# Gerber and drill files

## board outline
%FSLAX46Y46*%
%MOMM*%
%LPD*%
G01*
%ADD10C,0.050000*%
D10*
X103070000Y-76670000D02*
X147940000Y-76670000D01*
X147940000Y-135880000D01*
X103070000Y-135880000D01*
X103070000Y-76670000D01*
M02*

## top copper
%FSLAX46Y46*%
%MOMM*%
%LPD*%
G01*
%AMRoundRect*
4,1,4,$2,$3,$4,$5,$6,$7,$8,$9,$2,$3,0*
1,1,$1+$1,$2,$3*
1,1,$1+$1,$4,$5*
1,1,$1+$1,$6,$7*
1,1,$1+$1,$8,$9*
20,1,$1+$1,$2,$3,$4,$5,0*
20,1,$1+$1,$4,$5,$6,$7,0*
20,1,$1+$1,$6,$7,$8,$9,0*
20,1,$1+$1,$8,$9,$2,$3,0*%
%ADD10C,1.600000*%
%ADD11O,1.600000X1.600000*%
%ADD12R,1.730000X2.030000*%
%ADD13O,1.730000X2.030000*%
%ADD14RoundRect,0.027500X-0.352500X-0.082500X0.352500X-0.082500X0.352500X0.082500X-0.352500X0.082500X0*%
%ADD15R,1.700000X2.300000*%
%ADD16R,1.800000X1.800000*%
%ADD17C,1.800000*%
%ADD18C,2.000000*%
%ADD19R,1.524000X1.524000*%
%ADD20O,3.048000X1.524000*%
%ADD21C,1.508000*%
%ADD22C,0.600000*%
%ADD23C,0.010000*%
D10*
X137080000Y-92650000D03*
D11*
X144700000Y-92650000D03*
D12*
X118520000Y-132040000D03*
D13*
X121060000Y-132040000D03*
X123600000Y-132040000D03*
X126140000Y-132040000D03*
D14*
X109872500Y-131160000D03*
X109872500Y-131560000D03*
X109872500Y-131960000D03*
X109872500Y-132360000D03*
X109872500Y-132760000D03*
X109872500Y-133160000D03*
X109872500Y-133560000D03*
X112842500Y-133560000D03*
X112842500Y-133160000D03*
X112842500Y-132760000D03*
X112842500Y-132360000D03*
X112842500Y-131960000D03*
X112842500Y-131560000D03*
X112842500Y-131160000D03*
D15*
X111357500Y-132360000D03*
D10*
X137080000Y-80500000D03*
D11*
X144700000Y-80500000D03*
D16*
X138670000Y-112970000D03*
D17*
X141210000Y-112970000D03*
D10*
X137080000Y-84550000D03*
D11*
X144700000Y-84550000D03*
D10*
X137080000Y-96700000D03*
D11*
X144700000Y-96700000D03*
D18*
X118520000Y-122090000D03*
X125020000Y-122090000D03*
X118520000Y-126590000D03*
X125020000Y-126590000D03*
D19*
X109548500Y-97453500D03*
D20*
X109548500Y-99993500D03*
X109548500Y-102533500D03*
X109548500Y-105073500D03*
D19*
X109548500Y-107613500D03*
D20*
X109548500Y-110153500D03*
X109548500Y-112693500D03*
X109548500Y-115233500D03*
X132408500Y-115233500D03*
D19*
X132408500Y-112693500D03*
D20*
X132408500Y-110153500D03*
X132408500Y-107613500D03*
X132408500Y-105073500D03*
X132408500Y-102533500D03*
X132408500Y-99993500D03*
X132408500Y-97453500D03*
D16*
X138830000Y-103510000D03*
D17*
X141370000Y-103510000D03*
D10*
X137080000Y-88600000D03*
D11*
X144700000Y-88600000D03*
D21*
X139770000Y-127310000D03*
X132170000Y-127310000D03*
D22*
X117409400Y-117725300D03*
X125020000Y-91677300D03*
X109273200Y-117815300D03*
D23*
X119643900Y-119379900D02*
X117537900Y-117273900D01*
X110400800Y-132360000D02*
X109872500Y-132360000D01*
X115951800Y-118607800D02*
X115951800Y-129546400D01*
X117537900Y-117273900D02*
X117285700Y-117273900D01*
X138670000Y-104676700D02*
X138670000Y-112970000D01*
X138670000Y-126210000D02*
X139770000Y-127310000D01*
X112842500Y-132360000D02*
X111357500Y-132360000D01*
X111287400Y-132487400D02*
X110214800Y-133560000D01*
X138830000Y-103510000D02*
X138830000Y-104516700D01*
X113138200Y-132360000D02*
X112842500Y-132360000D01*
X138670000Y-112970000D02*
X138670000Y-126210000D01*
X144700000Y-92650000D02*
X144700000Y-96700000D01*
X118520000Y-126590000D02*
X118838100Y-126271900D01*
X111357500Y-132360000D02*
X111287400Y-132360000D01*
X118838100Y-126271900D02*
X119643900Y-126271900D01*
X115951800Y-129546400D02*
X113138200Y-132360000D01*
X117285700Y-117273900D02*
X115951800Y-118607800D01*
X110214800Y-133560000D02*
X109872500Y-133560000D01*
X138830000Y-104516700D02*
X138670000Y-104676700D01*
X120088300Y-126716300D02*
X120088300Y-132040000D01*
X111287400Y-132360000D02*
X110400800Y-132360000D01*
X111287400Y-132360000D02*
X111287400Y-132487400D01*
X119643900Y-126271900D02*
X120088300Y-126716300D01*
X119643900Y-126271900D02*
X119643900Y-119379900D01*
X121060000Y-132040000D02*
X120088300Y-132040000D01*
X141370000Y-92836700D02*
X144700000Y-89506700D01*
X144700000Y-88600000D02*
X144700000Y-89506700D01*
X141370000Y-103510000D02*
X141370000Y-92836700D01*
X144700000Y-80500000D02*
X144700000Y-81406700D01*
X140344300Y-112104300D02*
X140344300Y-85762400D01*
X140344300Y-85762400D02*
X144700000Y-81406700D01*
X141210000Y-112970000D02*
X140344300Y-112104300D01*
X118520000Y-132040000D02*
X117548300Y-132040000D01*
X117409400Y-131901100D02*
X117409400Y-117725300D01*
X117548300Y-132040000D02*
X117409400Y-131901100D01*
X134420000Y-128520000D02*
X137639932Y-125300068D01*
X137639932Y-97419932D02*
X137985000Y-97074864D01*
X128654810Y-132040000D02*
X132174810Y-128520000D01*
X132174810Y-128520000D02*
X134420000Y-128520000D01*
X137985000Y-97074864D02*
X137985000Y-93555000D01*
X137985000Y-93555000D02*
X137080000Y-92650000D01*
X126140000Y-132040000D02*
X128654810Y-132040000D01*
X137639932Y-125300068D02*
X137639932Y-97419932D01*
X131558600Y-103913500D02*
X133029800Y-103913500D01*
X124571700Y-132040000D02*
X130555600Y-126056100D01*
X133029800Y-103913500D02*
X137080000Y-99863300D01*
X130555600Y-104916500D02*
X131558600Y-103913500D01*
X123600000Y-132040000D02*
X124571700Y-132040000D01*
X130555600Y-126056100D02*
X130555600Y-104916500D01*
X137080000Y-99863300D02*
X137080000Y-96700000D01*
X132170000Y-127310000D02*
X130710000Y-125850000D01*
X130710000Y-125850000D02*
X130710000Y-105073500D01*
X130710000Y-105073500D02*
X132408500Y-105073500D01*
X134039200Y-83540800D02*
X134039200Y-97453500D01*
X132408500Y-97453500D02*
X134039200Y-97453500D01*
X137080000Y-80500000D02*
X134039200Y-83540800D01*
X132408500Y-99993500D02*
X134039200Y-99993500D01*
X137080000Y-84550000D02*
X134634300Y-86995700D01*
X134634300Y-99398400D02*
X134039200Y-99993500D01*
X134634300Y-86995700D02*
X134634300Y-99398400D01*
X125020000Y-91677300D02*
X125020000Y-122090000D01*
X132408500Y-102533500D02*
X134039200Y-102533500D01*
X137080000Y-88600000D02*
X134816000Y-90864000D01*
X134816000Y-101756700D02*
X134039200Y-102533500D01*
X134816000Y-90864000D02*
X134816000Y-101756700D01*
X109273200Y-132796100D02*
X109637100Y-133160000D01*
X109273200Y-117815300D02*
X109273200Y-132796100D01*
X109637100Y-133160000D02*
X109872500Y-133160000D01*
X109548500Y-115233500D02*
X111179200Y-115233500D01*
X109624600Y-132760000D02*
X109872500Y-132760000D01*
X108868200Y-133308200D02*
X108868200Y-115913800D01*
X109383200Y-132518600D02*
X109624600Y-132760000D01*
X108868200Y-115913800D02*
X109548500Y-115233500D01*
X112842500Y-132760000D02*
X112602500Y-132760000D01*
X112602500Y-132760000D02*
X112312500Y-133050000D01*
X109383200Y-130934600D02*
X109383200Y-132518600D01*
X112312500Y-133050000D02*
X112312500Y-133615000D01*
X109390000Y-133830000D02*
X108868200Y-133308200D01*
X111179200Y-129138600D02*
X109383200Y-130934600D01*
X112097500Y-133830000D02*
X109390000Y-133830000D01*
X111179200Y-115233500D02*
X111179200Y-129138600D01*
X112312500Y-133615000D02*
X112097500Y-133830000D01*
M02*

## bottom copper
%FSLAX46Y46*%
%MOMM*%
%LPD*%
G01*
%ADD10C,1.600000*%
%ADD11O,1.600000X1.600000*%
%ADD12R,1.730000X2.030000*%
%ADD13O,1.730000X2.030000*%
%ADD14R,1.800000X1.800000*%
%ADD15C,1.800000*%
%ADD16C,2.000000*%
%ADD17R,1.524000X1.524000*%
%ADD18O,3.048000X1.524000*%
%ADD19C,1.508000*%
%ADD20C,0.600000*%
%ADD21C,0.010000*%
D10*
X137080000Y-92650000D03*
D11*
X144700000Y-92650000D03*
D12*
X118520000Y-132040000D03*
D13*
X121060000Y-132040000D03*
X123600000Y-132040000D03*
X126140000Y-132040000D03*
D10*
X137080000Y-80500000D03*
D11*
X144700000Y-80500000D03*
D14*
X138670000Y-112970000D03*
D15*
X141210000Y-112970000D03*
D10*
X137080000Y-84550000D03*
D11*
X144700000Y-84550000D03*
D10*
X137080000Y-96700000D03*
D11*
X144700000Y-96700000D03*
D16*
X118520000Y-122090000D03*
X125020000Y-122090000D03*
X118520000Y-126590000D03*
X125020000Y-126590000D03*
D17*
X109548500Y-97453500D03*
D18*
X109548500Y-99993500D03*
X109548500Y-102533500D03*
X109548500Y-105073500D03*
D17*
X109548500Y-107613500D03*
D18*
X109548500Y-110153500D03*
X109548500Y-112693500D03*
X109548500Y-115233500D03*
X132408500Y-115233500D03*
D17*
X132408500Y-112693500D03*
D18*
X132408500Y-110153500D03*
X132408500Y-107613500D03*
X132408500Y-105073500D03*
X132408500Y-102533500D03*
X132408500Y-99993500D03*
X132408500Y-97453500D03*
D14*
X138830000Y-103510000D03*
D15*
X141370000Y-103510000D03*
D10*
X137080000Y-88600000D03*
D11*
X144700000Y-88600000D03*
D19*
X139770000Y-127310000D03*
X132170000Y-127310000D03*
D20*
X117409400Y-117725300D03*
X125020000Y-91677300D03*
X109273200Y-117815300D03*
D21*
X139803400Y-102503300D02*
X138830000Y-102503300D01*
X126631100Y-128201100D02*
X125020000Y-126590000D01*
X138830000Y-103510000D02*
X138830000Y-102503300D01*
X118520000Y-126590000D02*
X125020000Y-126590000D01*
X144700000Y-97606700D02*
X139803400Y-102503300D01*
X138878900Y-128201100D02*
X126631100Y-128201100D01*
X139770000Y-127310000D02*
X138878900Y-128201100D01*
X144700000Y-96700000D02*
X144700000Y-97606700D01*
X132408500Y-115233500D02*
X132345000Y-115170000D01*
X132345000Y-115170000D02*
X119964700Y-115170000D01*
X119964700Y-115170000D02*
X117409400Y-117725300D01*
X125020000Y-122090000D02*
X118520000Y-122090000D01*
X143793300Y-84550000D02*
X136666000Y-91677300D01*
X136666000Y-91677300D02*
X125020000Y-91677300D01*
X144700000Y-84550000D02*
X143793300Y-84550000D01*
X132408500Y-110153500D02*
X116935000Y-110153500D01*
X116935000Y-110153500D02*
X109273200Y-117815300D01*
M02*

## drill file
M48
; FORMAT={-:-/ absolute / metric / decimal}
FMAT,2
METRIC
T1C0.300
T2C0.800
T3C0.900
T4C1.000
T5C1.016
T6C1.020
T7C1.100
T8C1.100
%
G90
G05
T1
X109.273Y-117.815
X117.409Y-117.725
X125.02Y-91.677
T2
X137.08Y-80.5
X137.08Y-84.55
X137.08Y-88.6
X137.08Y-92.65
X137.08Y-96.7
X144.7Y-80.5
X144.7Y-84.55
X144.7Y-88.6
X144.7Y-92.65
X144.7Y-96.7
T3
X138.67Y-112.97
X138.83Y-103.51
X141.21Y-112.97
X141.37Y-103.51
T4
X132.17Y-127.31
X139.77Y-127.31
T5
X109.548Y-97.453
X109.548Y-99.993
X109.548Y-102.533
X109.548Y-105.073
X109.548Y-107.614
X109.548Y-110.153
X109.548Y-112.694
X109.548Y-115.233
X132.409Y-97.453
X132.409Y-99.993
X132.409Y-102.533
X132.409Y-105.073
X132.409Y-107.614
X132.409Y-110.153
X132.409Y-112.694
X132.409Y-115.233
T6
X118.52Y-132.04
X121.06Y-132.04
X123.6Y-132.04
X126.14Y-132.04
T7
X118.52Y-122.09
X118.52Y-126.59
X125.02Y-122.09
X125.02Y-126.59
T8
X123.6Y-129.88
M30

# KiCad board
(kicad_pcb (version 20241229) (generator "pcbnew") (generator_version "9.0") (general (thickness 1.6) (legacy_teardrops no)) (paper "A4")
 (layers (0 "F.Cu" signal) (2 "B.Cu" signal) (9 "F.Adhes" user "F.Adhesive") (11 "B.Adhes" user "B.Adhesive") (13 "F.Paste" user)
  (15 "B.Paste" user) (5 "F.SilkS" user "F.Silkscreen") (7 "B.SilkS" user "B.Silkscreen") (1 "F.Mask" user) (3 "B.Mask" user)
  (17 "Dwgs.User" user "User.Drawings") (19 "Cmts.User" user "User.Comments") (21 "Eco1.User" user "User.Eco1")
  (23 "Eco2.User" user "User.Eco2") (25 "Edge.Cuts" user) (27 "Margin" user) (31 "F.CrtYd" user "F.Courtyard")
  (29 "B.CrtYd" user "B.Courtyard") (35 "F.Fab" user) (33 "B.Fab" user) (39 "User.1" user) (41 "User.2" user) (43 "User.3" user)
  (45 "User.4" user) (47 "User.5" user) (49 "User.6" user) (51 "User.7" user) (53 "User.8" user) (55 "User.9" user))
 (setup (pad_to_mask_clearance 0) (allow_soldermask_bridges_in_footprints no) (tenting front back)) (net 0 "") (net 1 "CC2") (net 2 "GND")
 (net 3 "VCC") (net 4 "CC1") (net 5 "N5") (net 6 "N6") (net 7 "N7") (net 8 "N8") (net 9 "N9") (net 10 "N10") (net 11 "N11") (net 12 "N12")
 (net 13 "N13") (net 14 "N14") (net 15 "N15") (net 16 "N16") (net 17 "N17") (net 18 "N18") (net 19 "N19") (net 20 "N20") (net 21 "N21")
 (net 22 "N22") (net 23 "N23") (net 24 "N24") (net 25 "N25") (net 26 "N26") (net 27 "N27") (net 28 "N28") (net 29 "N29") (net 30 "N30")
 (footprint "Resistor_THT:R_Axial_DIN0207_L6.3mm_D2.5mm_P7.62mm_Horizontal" (layer "F.Cu") (at 137.08 92.65)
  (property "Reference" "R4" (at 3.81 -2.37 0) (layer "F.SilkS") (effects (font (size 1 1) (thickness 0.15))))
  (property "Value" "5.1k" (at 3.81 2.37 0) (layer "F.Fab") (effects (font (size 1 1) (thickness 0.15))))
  (pad "1" thru_hole circle (at 0 0) (size 1.6 1.6) (drill 0.8) (layers "*.Cu" "*.Mask") (remove_unused_layers no) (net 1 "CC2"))
  (pad "2" thru_hole oval (at 7.62 0) (size 1.6 1.6) (drill 0.8) (layers "*.Cu" "*.Mask") (remove_unused_layers no) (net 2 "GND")))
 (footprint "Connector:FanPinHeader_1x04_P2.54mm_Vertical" (layer "F.Cu") (at 118.52 132.04)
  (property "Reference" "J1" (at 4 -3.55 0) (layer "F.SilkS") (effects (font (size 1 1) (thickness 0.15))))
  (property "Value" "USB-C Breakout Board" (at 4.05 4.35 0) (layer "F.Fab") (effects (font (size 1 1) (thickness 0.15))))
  (pad "" np_thru_hole circle (at 5.08 -2.16 90) (size 1.1 1.1) (drill 1.1) (layers "*.Cu" "*.Mask"))
  (pad "1" thru_hole rect (at 0 0 90) (size 2.03 1.73) (drill 1.02) (layers "*.Cu" "*.Mask") (remove_unused_layers no) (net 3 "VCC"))
  (pad "2" thru_hole oval (at 2.54 0 90) (size 2.03 1.73) (drill 1.02) (layers "*.Cu" "*.Mask") (remove_unused_layers no) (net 2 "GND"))
  (pad "3" thru_hole oval (at 5.08 0 90) (size 2.03 1.73) (drill 1.02) (layers "*.Cu" "*.Mask") (remove_unused_layers no) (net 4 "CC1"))
  (pad "4" thru_hole oval (at 7.62 0 90) (size 2.03 1.73) (drill 1.02) (layers "*.Cu" "*.Mask") (remove_unused_layers no) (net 1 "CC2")))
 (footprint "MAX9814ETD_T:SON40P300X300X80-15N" (layer "F.Cu") (at 111.3575 132.36)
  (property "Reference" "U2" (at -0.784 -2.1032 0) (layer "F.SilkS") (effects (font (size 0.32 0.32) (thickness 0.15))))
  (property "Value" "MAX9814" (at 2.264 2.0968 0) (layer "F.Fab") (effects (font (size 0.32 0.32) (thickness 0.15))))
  (pad "1" smd roundrect (at -1.485 -1.2) (size 0.76 0.22) (layers "F.Cu" "F.Mask" "F.Paste") (roundrect_rratio 0.125) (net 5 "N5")
   (solder_mask_margin 0.102))
  (pad "2" smd roundrect (at -1.485 -0.8) (size 0.76 0.22) (layers "F.Cu" "F.Mask" "F.Paste") (roundrect_rratio 0.125) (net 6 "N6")
   (solder_mask_margin 0.102))
  (pad "3" smd roundrect (at -1.485 -0.4) (size 0.76 0.22) (layers "F.Cu" "F.Mask" "F.Paste") (roundrect_rratio 0.125) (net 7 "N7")
   (solder_mask_margin 0.102))
  (pad "4" smd roundrect (at -1.485 0) (size 0.76 0.22) (layers "F.Cu" "F.Mask" "F.Paste") (roundrect_rratio 0.125) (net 2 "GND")
   (solder_mask_margin 0.102))
  (pad "5" smd roundrect (at -1.485 0.4) (size 0.76 0.22) (layers "F.Cu" "F.Mask" "F.Paste") (roundrect_rratio 0.125) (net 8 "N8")
   (solder_mask_margin 0.102))
  (pad "6" smd roundrect (at -1.485 0.8) (size 0.76 0.22) (layers "F.Cu" "F.Mask" "F.Paste") (roundrect_rratio 0.125) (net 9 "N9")
   (solder_mask_margin 0.102))
  (pad "7" smd roundrect (at -1.485 1.2) (size 0.76 0.22) (layers "F.Cu" "F.Mask" "F.Paste") (roundrect_rratio 0.125) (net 2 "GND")
   (solder_mask_margin 0.102))
  (pad "8" smd roundrect (at 1.485 1.2) (size 0.76 0.22) (layers "F.Cu" "F.Mask" "F.Paste") (roundrect_rratio 0.125) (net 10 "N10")
   (solder_mask_margin 0.102))
  (pad "9" smd roundrect (at 1.485 0.8) (size 0.76 0.22) (layers "F.Cu" "F.Mask" "F.Paste") (roundrect_rratio 0.125) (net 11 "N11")
   (solder_mask_margin 0.102))
  (pad "10" smd roundrect (at 1.485 0.4) (size 0.76 0.22) (layers "F.Cu" "F.Mask" "F.Paste") (roundrect_rratio 0.125) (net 8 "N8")
   (solder_mask_margin 0.102))
  (pad "11" smd roundrect (at 1.485 0) (size 0.76 0.22) (layers "F.Cu" "F.Mask" "F.Paste") (roundrect_rratio 0.125) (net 2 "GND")
   (solder_mask_margin 0.102))
  (pad "12" smd roundrect (at 1.485 -0.4) (size 0.76 0.22) (layers "F.Cu" "F.Mask" "F.Paste") (roundrect_rratio 0.125) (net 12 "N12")
   (solder_mask_margin 0.102))
  (pad "13" smd roundrect (at 1.485 -0.8) (size 0.76 0.22) (layers "F.Cu" "F.Mask" "F.Paste") (roundrect_rratio 0.125) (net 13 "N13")
   (solder_mask_margin 0.102))
  (pad "14" smd roundrect (at 1.485 -1.2) (size 0.76 0.22) (layers "F.Cu" "F.Mask" "F.Paste") (roundrect_rratio 0.125) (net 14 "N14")
   (solder_mask_margin 0.102))
  (pad "15" smd rect (at 0 0) (size 1.7 2.3) (layers "F.Cu" "F.Mask") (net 2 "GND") (solder_mask_margin 0.102)))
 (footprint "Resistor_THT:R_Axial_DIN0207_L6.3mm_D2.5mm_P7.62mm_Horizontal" (layer "F.Cu") (at 137.08 80.5)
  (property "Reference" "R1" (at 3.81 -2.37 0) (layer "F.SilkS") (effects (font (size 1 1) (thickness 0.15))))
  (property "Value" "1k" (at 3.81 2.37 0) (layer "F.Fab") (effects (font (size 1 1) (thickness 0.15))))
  (pad "1" thru_hole circle (at 0 0) (size 1.6 1.6) (drill 0.8) (layers "*.Cu" "*.Mask") (remove_unused_layers no) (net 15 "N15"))
  (pad "2" thru_hole oval (at 7.62 0) (size 1.6 1.6) (drill 0.8) (layers "*.Cu" "*.Mask") (remove_unused_layers no) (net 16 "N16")))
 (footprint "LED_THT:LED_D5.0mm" (layer "F.Cu") (at 138.67 112.97)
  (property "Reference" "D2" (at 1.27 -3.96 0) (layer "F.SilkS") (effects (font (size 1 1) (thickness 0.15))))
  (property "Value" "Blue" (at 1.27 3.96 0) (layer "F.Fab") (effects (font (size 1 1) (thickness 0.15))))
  (pad "1" thru_hole rect (at 0 0) (size 1.8 1.8) (drill 0.9) (layers "*.Cu" "*.Mask") (remove_unused_layers no) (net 2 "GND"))
  (pad "2" thru_hole circle (at 2.54 0) (size 1.8 1.8) (drill 0.9) (layers "*.Cu" "*.Mask") (remove_unused_layers no) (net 16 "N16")))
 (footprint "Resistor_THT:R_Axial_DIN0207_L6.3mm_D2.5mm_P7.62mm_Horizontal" (layer "F.Cu") (at 137.08 84.55)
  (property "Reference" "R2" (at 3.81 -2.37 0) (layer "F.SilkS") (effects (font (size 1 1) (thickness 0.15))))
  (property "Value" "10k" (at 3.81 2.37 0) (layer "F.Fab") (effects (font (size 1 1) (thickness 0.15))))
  (pad "1" thru_hole circle (at 0 0) (size 1.6 1.6) (drill 0.8) (layers "*.Cu" "*.Mask") (remove_unused_layers no) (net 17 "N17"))
  (pad "2" thru_hole oval (at 7.62 0) (size 1.6 1.6) (drill 0.8) (layers "*.Cu" "*.Mask") (remove_unused_layers no) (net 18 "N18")))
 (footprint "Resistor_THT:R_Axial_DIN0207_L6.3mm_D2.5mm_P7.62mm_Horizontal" (layer "F.Cu") (at 137.08 96.7)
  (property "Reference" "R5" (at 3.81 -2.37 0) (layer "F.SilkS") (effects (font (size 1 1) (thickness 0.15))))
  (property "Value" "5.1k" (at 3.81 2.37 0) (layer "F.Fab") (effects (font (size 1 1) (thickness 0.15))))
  (pad "1" thru_hole circle (at 0 0) (size 1.6 1.6) (drill 0.8) (layers "*.Cu" "*.Mask") (remove_unused_layers no) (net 4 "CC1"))
  (pad "2" thru_hole oval (at 7.62 0) (size 1.6 1.6) (drill 0.8) (layers "*.Cu" "*.Mask") (remove_unused_layers no) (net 2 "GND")))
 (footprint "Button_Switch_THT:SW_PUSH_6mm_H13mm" (layer "F.Cu") (at 118.52 122.09)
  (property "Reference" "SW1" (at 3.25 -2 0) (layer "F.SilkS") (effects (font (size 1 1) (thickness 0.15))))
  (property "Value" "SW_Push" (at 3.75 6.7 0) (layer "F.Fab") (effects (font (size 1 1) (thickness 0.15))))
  (pad "1" thru_hole circle (at 0 0 90) (size 2 2) (drill 1.1) (layers "*.Cu" "*.Mask") (remove_unused_layers no) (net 18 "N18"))
  (pad "1" thru_hole circle (at 6.5 0 90) (size 2 2) (drill 1.1) (layers "*.Cu" "*.Mask") (remove_unused_layers no) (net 18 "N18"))
  (pad "2" thru_hole circle (at 0 4.5 90) (size 2 2) (drill 1.1) (layers "*.Cu" "*.Mask") (remove_unused_layers no) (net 2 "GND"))
  (pad "2" thru_hole circle (at 6.5 4.5 90) (size 2 2) (drill 1.1) (layers "*.Cu" "*.Mask") (remove_unused_layers no) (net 2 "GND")))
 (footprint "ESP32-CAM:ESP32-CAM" (layer "F.Cu") (at 120.9785 105.0735)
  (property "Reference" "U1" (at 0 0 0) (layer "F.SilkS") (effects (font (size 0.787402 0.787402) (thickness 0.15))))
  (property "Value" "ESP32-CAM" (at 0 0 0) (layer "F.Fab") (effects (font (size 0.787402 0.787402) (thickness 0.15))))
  (pad "P$1" thru_hole rect (at -11.43 -7.62) (size 1.524 1.524) (drill 1.016) (layers "*.Cu" "*.Mask") (remove_unused_layers no)
   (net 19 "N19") (solder_mask_margin 0.102))
  (pad "P$2" thru_hole oval (at -11.43 -5.08) (size 3.048 1.524) (drill 1.016) (layers "*.Cu" "*.Mask") (remove_unused_layers no)
   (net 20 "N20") (solder_mask_margin 0.102))
  (pad "P$3" thru_hole oval (at -11.43 -2.54) (size 3.048 1.524) (drill 1.016) (layers "*.Cu" "*.Mask") (remove_unused_layers no)
   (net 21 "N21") (solder_mask_margin 0.102))
  (pad "P$4" thru_hole oval (at -11.43 0) (size 3.048 1.524) (drill 1.016) (layers "*.Cu" "*.Mask") (remove_unused_layers no) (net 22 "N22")
   (solder_mask_margin 0.102))
  (pad "P$5" thru_hole rect (at -11.43 2.54) (size 1.524 1.524) (drill 1.016) (layers "*.Cu" "*.Mask") (remove_unused_layers no)
   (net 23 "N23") (solder_mask_margin 0.102))
  (pad "P$6" thru_hole oval (at -11.43 5.08) (size 3.048 1.524) (drill 1.016) (layers "*.Cu" "*.Mask") (remove_unused_layers no)
   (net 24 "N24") (solder_mask_margin 0.102))
  (pad "P$7" thru_hole oval (at -11.43 7.62) (size 3.048 1.524) (drill 1.016) (layers "*.Cu" "*.Mask") (remove_unused_layers no)
   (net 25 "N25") (solder_mask_margin 0.102))
  (pad "P$8" thru_hole oval (at -11.43 10.16) (size 3.048 1.524) (drill 1.016) (layers "*.Cu" "*.Mask") (remove_unused_layers no)
   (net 8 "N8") (solder_mask_margin 0.102))
  (pad "P$9" thru_hole oval (at 11.43 10.16) (size 3.048 1.524) (drill 1.016) (layers "*.Cu" "*.Mask") (remove_unused_layers no)
   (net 3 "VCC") (solder_mask_margin 0.102))
  (pad "P$10" thru_hole rect (at 11.43 7.62) (size 1.524 1.524) (drill 1.016) (layers "*.Cu" "*.Mask") (remove_unused_layers no)
   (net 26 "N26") (solder_mask_margin 0.102))
  (pad "P$11" thru_hole oval (at 11.43 5.08) (size 3.048 1.524) (drill 1.016) (layers "*.Cu" "*.Mask") (remove_unused_layers no)
   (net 9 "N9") (solder_mask_margin 0.102))
  (pad "P$12" thru_hole oval (at 11.43 2.54) (size 3.048 1.524) (drill 1.016) (layers "*.Cu" "*.Mask") (remove_unused_layers no)
   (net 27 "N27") (solder_mask_margin 0.102))
  (pad "P$13" thru_hole oval (at 11.43 0) (size 3.048 1.524) (drill 1.016) (layers "*.Cu" "*.Mask") (remove_unused_layers no) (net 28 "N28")
   (solder_mask_margin 0.102))
  (pad "P$14" thru_hole oval (at 11.43 -2.54) (size 3.048 1.524) (drill 1.016) (layers "*.Cu" "*.Mask") (remove_unused_layers no)
   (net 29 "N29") (solder_mask_margin 0.102))
  (pad "P$15" thru_hole oval (at 11.43 -5.08) (size 3.048 1.524) (drill 1.016) (layers "*.Cu" "*.Mask") (remove_unused_layers no)
   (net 17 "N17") (solder_mask_margin 0.102))
  (pad "P$16" thru_hole oval (at 11.43 -7.62) (size 3.048 1.524) (drill 1.016) (layers "*.Cu" "*.Mask") (remove_unused_layers no)
   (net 15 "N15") (solder_mask_margin 0.102)))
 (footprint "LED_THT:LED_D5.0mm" (layer "F.Cu") (at 138.83 103.51)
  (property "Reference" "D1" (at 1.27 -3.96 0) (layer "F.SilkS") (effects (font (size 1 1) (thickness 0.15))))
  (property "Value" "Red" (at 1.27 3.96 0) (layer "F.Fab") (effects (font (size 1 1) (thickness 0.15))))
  (pad "1" thru_hole rect (at 0 0) (size 1.8 1.8) (drill 0.9) (layers "*.Cu" "*.Mask") (remove_unused_layers no) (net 2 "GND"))
  (pad "2" thru_hole circle (at 2.54 0) (size 1.8 1.8) (drill 0.9) (layers "*.Cu" "*.Mask") (remove_unused_layers no) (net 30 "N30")))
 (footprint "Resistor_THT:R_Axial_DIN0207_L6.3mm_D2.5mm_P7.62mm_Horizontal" (layer "F.Cu") (at 137.08 88.6)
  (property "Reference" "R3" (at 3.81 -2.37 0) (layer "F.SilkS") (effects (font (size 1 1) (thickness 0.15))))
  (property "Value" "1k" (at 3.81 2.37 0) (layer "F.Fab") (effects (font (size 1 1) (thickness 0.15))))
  (pad "1" thru_hole circle (at 0 0) (size 1.6 1.6) (drill 0.8) (layers "*.Cu" "*.Mask") (remove_unused_layers no) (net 29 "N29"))
  (pad "2" thru_hole oval (at 7.62 0) (size 1.6 1.6) (drill 0.8) (layers "*.Cu" "*.Mask") (remove_unused_layers no) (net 30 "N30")))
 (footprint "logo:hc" (layer "F.Cu") (at 121 89)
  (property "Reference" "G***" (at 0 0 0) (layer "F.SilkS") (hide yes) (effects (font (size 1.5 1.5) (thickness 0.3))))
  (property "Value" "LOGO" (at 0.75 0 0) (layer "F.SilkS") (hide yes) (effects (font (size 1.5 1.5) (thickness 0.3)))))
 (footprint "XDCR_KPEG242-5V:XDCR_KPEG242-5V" (layer "F.Cu") (at 135.97 127.31)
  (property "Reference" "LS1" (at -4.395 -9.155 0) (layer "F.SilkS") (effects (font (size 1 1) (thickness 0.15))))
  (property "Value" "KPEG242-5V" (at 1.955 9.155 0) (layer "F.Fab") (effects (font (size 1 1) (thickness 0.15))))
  (pad "N" thru_hole circle (at 3.8 0) (size 1.508 1.508) (drill 1) (layers "*.Cu" "*.Mask") (remove_unused_layers no) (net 2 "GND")
   (solder_mask_margin 0.102))
  (pad "P" thru_hole circle (at -3.8 0) (size 1.508 1.508) (drill 1) (layers "*.Cu" "*.Mask") (remove_unused_layers no) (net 28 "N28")
   (solder_mask_margin 0.102)))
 (gr_rect (start 103.07 76.67) (end 147.94 135.88) (stroke (width 0.05) (type default)) (fill no) (layer "Edge.Cuts"))
 (segment (start 119.6439 119.3799) (end 117.5379 117.2739) (width 0.01) (layer "F.Cu") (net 2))
 (segment (start 110.4008 132.36) (end 109.8725 132.36) (width 0.01) (layer "F.Cu") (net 2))
 (segment (start 115.9518 118.6078) (end 115.9518 129.5464) (width 0.01) (layer "F.Cu") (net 2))
 (segment (start 117.5379 117.2739) (end 117.2857 117.2739) (width 0.01) (layer "F.Cu") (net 2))
 (segment (start 138.67 104.6767) (end 138.67 112.97) (width 0.01) (layer "F.Cu") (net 2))
 (segment (start 138.67 126.21) (end 139.77 127.31) (width 0.01) (layer "F.Cu") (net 2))
 (segment (start 112.8425 132.36) (end 111.3575 132.36) (width 0.01) (layer "F.Cu") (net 2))
 (segment (start 111.2874 132.4874) (end 110.2148 133.56) (width 0.01) (layer "F.Cu") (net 2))
 (segment (start 138.83 103.51) (end 138.83 104.5167) (width 0.01) (layer "F.Cu") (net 2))
 (segment (start 113.1382 132.36) (end 112.8425 132.36) (width 0.01) (layer "F.Cu") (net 2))
 (segment (start 138.67 112.97) (end 138.67 126.21) (width 0.01) (layer "F.Cu") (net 2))
 (segment (start 144.7 92.65) (end 144.7 96.7) (width 0.01) (layer "F.Cu") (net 2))
 (segment (start 118.52 126.59) (end 118.8381 126.2719) (width 0.01) (layer "F.Cu") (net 2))
 (segment (start 111.3575 132.36) (end 111.2874 132.36) (width 0.01) (layer "F.Cu") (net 2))
 (segment (start 118.8381 126.2719) (end 119.6439 126.2719) (width 0.01) (layer "F.Cu") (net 2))
 (segment (start 115.9518 129.5464) (end 113.1382 132.36) (width 0.01) (layer "F.Cu") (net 2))
 (segment (start 117.2857 117.2739) (end 115.9518 118.6078) (width 0.01) (layer "F.Cu") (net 2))
 (segment (start 110.2148 133.56) (end 109.8725 133.56) (width 0.01) (layer "F.Cu") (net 2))
 (segment (start 138.83 104.5167) (end 138.67 104.6767) (width 0.01) (layer "F.Cu") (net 2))
 (segment (start 120.0883 126.7163) (end 120.0883 132.04) (width 0.01) (layer "F.Cu") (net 2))
 (segment (start 111.2874 132.36) (end 110.4008 132.36) (width 0.01) (layer "F.Cu") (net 2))
 (segment (start 111.2874 132.36) (end 111.2874 132.4874) (width 0.01) (layer "F.Cu") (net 2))
 (segment (start 119.6439 126.2719) (end 120.0883 126.7163) (width 0.01) (layer "F.Cu") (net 2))
 (segment (start 119.6439 126.2719) (end 119.6439 119.3799) (width 0.01) (layer "F.Cu") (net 2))
 (segment (start 121.06 132.04) (end 120.0883 132.04) (width 0.01) (layer "F.Cu") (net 2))
 (segment (start 139.8034 102.5033) (end 138.83 102.5033) (width 0.01) (layer "B.Cu") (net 2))
 (segment (start 126.6311 128.2011) (end 125.02 126.59) (width 0.01) (layer "B.Cu") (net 2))
 (segment (start 138.83 103.51) (end 138.83 102.5033) (width 0.01) (layer "B.Cu") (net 2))
 (segment (start 118.52 126.59) (end 125.02 126.59) (width 0.01) (layer "B.Cu") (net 2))
 (segment (start 144.7 97.6067) (end 139.8034 102.5033) (width 0.01) (layer "B.Cu") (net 2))
 (segment (start 138.8789 128.2011) (end 126.6311 128.2011) (width 0.01) (layer "B.Cu") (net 2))
 (segment (start 139.77 127.31) (end 138.8789 128.2011) (width 0.01) (layer "B.Cu") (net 2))
 (segment (start 144.7 96.7) (end 144.7 97.6067) (width 0.01) (layer "B.Cu") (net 2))
 (segment (start 141.37 92.8367) (end 144.7 89.5067) (width 0.01) (layer "F.Cu") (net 30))
 (segment (start 144.7 88.6) (end 144.7 89.5067) (width 0.01) (layer "F.Cu") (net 30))
 (segment (start 141.37 103.51) (end 141.37 92.8367) (width 0.01) (layer "F.Cu") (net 30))
 (segment (start 144.7 80.5) (end 144.7 81.4067) (width 0.01) (layer "F.Cu") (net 16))
 (segment (start 140.3443 112.1043) (end 140.3443 85.7624) (width 0.01) (layer "F.Cu") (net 16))
 (segment (start 140.3443 85.7624) (end 144.7 81.4067) (width 0.01) (layer "F.Cu") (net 16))
 (segment (start 141.21 112.97) (end 140.3443 112.1043) (width 0.01) (layer "F.Cu") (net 16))
 (segment (start 118.52 132.04) (end 117.5483 132.04) (width 0.01) (layer "F.Cu") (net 3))
 (segment (start 117.4094 131.9011) (end 117.4094 117.7253) (width 0.01) (layer "F.Cu") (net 3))
 (segment (start 117.5483 132.04) (end 117.4094 131.9011) (width 0.01) (layer "F.Cu") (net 3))
 (via (at 117.4094 117.7253) (size 0.6) (drill 0.3) (layers "F.Cu" "B.Cu") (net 3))
 (segment (start 132.4085 115.2335) (end 132.345 115.17) (width 0.01) (layer "B.Cu") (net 3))
 (segment (start 132.345 115.17) (end 119.9647 115.17) (width 0.01) (layer "B.Cu") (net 3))
 (segment (start 119.9647 115.17) (end 117.4094 117.7253) (width 0.01) (layer "B.Cu") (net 3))
 (segment (start 134.42 128.52) (end 137.639932 125.300068) (width 0.01) (layer "F.Cu") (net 1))
 (segment (start 137.639932 97.419932) (end 137.985 97.074864) (width 0.01) (layer "F.Cu") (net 1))
 (segment (start 128.65481 132.04) (end 132.17481 128.52) (width 0.01) (layer "F.Cu") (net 1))
 (segment (start 132.17481 128.52) (end 134.42 128.52) (width 0.01) (layer "F.Cu") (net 1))
 (segment (start 137.985 97.074864) (end 137.985 93.555) (width 0.01) (layer "F.Cu") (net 1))
 (segment (start 137.985 93.555) (end 137.08 92.65) (width 0.01) (layer "F.Cu") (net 1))
 (segment (start 126.14 132.04) (end 128.65481 132.04) (width 0.01) (layer "F.Cu") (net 1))
 (segment (start 137.639932 125.300068) (end 137.639932 97.419932) (width 0.01) (layer "F.Cu") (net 1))
 (segment (start 131.5586 103.9135) (end 133.0298 103.9135) (width 0.01) (layer "F.Cu") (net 4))
 (segment (start 124.5717 132.04) (end 130.5556 126.0561) (width 0.01) (layer "F.Cu") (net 4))
 (segment (start 133.0298 103.9135) (end 137.08 99.8633) (width 0.01) (layer "F.Cu") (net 4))
 (segment (start 130.5556 104.9165) (end 131.5586 103.9135) (width 0.01) (layer "F.Cu") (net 4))
 (segment (start 123.6 132.04) (end 124.5717 132.04) (width 0.01) (layer "F.Cu") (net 4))
 (segment (start 130.5556 126.0561) (end 130.5556 104.9165) (width 0.01) (layer "F.Cu") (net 4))
 (segment (start 137.08 99.8633) (end 137.08 96.7) (width 0.01) (layer "F.Cu") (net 4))
 (segment (start 132.17 127.31) (end 130.71 125.85) (width 0.01) (layer "F.Cu") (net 28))
 (segment (start 130.71 125.85) (end 130.71 105.0735) (width 0.01) (layer "F.Cu") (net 28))
 (segment (start 130.71 105.0735) (end 132.4085 105.0735) (width 0.01) (layer "F.Cu") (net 28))
 (segment (start 134.0392 83.5408) (end 134.0392 97.4535) (width 0.01) (layer "F.Cu") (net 15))
 (segment (start 132.4085 97.4535) (end 134.0392 97.4535) (width 0.01) (layer "F.Cu") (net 15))
 (segment (start 137.08 80.5) (end 134.0392 83.5408) (width 0.01) (layer "F.Cu") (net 15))
 (segment (start 132.4085 99.9935) (end 134.0392 99.9935) (width 0.01) (layer "F.Cu") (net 17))
 (segment (start 137.08 84.55) (end 134.6343 86.9957) (width 0.01) (layer "F.Cu") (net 17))
 (segment (start 134.6343 99.3984) (end 134.0392 99.9935) (width 0.01) (layer "F.Cu") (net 17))
 (segment (start 134.6343 86.9957) (end 134.6343 99.3984) (width 0.01) (layer "F.Cu") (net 17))
 (segment (start 125.02 91.6773) (end 125.02 122.09) (width 0.01) (layer "F.Cu") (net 18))
 (via (at 125.02 91.6773) (size 0.6) (drill 0.3) (layers "F.Cu" "B.Cu") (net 18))
 (segment (start 125.02 122.09) (end 118.52 122.09) (width 0.01) (layer "B.Cu") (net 18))
 (segment (start 143.7933 84.55) (end 136.666 91.6773) (width 0.01) (layer "B.Cu") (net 18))
 (segment (start 136.666 91.6773) (end 125.02 91.6773) (width 0.01) (layer "B.Cu") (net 18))
 (segment (start 144.7 84.55) (end 143.7933 84.55) (width 0.01) (layer "B.Cu") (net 18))
 (segment (start 132.4085 102.5335) (end 134.0392 102.5335) (width 0.01) (layer "F.Cu") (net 29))
 (segment (start 137.08 88.6) (end 134.816 90.864) (width 0.01) (layer "F.Cu") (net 29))
 (segment (start 134.816 101.7567) (end 134.0392 102.5335) (width 0.01) (layer "F.Cu") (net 29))
 (segment (start 134.816 90.864) (end 134.816 101.7567) (width 0.01) (layer "F.Cu") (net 29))
 (segment (start 109.2732 132.7961) (end 109.6371 133.16) (width 0.01) (layer "F.Cu") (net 9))
 (segment (start 109.2732 117.8153) (end 109.2732 132.7961) (width 0.01) (layer "F.Cu") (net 9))
 (segment (start 109.6371 133.16) (end 109.8725 133.16) (width 0.01) (layer "F.Cu") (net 9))
 (via (at 109.2732 117.8153) (size 0.6) (drill 0.3) (layers "F.Cu" "B.Cu") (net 9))
 (segment (start 132.4085 110.1535) (end 116.935 110.1535) (width 0.01) (layer "B.Cu") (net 9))
 (segment (start 116.935 110.1535) (end 109.2732 117.8153) (width 0.01) (layer "B.Cu") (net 9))
 (segment (start 109.5485 115.2335) (end 111.1792 115.2335) (width 0.01) (layer "F.Cu") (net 8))
 (segment (start 109.6246 132.76) (end 109.8725 132.76) (width 0.01) (layer "F.Cu") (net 8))
 (segment (start 108.8682 133.3082) (end 108.8682 115.9138) (width 0.01) (layer "F.Cu") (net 8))
 (segment (start 109.3832 132.5186) (end 109.6246 132.76) (width 0.01) (layer "F.Cu") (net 8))
 (segment (start 108.8682 115.9138) (end 109.5485 115.2335) (width 0.01) (layer "F.Cu") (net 8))
 (segment (start 112.8425 132.76) (end 112.6025 132.76) (width 0.01) (layer "F.Cu") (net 8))
 (segment (start 112.6025 132.76) (end 112.3125 133.05) (width 0.01) (layer "F.Cu") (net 8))
 (segment (start 109.3832 130.9346) (end 109.3832 132.5186) (width 0.01) (layer "F.Cu") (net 8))
 (segment (start 112.3125 133.05) (end 112.3125 133.615) (width 0.01) (layer "F.Cu") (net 8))
 (segment (start 109.39 133.83) (end 108.8682 133.3082) (width 0.01) (layer "F.Cu") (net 8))
 (segment (start 111.1792 129.1386) (end 109.3832 130.9346) (width 0.01) (layer "F.Cu") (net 8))
 (segment (start 112.0975 133.83) (end 109.39 133.83) (width 0.01) (layer "F.Cu") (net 8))
 (segment (start 111.1792 115.2335) (end 111.1792 129.1386) (width 0.01) (layer "F.Cu") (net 8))
 (segment (start 112.3125 133.615) (end 112.0975 133.83) (width 0.01) (layer "F.Cu") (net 8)))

